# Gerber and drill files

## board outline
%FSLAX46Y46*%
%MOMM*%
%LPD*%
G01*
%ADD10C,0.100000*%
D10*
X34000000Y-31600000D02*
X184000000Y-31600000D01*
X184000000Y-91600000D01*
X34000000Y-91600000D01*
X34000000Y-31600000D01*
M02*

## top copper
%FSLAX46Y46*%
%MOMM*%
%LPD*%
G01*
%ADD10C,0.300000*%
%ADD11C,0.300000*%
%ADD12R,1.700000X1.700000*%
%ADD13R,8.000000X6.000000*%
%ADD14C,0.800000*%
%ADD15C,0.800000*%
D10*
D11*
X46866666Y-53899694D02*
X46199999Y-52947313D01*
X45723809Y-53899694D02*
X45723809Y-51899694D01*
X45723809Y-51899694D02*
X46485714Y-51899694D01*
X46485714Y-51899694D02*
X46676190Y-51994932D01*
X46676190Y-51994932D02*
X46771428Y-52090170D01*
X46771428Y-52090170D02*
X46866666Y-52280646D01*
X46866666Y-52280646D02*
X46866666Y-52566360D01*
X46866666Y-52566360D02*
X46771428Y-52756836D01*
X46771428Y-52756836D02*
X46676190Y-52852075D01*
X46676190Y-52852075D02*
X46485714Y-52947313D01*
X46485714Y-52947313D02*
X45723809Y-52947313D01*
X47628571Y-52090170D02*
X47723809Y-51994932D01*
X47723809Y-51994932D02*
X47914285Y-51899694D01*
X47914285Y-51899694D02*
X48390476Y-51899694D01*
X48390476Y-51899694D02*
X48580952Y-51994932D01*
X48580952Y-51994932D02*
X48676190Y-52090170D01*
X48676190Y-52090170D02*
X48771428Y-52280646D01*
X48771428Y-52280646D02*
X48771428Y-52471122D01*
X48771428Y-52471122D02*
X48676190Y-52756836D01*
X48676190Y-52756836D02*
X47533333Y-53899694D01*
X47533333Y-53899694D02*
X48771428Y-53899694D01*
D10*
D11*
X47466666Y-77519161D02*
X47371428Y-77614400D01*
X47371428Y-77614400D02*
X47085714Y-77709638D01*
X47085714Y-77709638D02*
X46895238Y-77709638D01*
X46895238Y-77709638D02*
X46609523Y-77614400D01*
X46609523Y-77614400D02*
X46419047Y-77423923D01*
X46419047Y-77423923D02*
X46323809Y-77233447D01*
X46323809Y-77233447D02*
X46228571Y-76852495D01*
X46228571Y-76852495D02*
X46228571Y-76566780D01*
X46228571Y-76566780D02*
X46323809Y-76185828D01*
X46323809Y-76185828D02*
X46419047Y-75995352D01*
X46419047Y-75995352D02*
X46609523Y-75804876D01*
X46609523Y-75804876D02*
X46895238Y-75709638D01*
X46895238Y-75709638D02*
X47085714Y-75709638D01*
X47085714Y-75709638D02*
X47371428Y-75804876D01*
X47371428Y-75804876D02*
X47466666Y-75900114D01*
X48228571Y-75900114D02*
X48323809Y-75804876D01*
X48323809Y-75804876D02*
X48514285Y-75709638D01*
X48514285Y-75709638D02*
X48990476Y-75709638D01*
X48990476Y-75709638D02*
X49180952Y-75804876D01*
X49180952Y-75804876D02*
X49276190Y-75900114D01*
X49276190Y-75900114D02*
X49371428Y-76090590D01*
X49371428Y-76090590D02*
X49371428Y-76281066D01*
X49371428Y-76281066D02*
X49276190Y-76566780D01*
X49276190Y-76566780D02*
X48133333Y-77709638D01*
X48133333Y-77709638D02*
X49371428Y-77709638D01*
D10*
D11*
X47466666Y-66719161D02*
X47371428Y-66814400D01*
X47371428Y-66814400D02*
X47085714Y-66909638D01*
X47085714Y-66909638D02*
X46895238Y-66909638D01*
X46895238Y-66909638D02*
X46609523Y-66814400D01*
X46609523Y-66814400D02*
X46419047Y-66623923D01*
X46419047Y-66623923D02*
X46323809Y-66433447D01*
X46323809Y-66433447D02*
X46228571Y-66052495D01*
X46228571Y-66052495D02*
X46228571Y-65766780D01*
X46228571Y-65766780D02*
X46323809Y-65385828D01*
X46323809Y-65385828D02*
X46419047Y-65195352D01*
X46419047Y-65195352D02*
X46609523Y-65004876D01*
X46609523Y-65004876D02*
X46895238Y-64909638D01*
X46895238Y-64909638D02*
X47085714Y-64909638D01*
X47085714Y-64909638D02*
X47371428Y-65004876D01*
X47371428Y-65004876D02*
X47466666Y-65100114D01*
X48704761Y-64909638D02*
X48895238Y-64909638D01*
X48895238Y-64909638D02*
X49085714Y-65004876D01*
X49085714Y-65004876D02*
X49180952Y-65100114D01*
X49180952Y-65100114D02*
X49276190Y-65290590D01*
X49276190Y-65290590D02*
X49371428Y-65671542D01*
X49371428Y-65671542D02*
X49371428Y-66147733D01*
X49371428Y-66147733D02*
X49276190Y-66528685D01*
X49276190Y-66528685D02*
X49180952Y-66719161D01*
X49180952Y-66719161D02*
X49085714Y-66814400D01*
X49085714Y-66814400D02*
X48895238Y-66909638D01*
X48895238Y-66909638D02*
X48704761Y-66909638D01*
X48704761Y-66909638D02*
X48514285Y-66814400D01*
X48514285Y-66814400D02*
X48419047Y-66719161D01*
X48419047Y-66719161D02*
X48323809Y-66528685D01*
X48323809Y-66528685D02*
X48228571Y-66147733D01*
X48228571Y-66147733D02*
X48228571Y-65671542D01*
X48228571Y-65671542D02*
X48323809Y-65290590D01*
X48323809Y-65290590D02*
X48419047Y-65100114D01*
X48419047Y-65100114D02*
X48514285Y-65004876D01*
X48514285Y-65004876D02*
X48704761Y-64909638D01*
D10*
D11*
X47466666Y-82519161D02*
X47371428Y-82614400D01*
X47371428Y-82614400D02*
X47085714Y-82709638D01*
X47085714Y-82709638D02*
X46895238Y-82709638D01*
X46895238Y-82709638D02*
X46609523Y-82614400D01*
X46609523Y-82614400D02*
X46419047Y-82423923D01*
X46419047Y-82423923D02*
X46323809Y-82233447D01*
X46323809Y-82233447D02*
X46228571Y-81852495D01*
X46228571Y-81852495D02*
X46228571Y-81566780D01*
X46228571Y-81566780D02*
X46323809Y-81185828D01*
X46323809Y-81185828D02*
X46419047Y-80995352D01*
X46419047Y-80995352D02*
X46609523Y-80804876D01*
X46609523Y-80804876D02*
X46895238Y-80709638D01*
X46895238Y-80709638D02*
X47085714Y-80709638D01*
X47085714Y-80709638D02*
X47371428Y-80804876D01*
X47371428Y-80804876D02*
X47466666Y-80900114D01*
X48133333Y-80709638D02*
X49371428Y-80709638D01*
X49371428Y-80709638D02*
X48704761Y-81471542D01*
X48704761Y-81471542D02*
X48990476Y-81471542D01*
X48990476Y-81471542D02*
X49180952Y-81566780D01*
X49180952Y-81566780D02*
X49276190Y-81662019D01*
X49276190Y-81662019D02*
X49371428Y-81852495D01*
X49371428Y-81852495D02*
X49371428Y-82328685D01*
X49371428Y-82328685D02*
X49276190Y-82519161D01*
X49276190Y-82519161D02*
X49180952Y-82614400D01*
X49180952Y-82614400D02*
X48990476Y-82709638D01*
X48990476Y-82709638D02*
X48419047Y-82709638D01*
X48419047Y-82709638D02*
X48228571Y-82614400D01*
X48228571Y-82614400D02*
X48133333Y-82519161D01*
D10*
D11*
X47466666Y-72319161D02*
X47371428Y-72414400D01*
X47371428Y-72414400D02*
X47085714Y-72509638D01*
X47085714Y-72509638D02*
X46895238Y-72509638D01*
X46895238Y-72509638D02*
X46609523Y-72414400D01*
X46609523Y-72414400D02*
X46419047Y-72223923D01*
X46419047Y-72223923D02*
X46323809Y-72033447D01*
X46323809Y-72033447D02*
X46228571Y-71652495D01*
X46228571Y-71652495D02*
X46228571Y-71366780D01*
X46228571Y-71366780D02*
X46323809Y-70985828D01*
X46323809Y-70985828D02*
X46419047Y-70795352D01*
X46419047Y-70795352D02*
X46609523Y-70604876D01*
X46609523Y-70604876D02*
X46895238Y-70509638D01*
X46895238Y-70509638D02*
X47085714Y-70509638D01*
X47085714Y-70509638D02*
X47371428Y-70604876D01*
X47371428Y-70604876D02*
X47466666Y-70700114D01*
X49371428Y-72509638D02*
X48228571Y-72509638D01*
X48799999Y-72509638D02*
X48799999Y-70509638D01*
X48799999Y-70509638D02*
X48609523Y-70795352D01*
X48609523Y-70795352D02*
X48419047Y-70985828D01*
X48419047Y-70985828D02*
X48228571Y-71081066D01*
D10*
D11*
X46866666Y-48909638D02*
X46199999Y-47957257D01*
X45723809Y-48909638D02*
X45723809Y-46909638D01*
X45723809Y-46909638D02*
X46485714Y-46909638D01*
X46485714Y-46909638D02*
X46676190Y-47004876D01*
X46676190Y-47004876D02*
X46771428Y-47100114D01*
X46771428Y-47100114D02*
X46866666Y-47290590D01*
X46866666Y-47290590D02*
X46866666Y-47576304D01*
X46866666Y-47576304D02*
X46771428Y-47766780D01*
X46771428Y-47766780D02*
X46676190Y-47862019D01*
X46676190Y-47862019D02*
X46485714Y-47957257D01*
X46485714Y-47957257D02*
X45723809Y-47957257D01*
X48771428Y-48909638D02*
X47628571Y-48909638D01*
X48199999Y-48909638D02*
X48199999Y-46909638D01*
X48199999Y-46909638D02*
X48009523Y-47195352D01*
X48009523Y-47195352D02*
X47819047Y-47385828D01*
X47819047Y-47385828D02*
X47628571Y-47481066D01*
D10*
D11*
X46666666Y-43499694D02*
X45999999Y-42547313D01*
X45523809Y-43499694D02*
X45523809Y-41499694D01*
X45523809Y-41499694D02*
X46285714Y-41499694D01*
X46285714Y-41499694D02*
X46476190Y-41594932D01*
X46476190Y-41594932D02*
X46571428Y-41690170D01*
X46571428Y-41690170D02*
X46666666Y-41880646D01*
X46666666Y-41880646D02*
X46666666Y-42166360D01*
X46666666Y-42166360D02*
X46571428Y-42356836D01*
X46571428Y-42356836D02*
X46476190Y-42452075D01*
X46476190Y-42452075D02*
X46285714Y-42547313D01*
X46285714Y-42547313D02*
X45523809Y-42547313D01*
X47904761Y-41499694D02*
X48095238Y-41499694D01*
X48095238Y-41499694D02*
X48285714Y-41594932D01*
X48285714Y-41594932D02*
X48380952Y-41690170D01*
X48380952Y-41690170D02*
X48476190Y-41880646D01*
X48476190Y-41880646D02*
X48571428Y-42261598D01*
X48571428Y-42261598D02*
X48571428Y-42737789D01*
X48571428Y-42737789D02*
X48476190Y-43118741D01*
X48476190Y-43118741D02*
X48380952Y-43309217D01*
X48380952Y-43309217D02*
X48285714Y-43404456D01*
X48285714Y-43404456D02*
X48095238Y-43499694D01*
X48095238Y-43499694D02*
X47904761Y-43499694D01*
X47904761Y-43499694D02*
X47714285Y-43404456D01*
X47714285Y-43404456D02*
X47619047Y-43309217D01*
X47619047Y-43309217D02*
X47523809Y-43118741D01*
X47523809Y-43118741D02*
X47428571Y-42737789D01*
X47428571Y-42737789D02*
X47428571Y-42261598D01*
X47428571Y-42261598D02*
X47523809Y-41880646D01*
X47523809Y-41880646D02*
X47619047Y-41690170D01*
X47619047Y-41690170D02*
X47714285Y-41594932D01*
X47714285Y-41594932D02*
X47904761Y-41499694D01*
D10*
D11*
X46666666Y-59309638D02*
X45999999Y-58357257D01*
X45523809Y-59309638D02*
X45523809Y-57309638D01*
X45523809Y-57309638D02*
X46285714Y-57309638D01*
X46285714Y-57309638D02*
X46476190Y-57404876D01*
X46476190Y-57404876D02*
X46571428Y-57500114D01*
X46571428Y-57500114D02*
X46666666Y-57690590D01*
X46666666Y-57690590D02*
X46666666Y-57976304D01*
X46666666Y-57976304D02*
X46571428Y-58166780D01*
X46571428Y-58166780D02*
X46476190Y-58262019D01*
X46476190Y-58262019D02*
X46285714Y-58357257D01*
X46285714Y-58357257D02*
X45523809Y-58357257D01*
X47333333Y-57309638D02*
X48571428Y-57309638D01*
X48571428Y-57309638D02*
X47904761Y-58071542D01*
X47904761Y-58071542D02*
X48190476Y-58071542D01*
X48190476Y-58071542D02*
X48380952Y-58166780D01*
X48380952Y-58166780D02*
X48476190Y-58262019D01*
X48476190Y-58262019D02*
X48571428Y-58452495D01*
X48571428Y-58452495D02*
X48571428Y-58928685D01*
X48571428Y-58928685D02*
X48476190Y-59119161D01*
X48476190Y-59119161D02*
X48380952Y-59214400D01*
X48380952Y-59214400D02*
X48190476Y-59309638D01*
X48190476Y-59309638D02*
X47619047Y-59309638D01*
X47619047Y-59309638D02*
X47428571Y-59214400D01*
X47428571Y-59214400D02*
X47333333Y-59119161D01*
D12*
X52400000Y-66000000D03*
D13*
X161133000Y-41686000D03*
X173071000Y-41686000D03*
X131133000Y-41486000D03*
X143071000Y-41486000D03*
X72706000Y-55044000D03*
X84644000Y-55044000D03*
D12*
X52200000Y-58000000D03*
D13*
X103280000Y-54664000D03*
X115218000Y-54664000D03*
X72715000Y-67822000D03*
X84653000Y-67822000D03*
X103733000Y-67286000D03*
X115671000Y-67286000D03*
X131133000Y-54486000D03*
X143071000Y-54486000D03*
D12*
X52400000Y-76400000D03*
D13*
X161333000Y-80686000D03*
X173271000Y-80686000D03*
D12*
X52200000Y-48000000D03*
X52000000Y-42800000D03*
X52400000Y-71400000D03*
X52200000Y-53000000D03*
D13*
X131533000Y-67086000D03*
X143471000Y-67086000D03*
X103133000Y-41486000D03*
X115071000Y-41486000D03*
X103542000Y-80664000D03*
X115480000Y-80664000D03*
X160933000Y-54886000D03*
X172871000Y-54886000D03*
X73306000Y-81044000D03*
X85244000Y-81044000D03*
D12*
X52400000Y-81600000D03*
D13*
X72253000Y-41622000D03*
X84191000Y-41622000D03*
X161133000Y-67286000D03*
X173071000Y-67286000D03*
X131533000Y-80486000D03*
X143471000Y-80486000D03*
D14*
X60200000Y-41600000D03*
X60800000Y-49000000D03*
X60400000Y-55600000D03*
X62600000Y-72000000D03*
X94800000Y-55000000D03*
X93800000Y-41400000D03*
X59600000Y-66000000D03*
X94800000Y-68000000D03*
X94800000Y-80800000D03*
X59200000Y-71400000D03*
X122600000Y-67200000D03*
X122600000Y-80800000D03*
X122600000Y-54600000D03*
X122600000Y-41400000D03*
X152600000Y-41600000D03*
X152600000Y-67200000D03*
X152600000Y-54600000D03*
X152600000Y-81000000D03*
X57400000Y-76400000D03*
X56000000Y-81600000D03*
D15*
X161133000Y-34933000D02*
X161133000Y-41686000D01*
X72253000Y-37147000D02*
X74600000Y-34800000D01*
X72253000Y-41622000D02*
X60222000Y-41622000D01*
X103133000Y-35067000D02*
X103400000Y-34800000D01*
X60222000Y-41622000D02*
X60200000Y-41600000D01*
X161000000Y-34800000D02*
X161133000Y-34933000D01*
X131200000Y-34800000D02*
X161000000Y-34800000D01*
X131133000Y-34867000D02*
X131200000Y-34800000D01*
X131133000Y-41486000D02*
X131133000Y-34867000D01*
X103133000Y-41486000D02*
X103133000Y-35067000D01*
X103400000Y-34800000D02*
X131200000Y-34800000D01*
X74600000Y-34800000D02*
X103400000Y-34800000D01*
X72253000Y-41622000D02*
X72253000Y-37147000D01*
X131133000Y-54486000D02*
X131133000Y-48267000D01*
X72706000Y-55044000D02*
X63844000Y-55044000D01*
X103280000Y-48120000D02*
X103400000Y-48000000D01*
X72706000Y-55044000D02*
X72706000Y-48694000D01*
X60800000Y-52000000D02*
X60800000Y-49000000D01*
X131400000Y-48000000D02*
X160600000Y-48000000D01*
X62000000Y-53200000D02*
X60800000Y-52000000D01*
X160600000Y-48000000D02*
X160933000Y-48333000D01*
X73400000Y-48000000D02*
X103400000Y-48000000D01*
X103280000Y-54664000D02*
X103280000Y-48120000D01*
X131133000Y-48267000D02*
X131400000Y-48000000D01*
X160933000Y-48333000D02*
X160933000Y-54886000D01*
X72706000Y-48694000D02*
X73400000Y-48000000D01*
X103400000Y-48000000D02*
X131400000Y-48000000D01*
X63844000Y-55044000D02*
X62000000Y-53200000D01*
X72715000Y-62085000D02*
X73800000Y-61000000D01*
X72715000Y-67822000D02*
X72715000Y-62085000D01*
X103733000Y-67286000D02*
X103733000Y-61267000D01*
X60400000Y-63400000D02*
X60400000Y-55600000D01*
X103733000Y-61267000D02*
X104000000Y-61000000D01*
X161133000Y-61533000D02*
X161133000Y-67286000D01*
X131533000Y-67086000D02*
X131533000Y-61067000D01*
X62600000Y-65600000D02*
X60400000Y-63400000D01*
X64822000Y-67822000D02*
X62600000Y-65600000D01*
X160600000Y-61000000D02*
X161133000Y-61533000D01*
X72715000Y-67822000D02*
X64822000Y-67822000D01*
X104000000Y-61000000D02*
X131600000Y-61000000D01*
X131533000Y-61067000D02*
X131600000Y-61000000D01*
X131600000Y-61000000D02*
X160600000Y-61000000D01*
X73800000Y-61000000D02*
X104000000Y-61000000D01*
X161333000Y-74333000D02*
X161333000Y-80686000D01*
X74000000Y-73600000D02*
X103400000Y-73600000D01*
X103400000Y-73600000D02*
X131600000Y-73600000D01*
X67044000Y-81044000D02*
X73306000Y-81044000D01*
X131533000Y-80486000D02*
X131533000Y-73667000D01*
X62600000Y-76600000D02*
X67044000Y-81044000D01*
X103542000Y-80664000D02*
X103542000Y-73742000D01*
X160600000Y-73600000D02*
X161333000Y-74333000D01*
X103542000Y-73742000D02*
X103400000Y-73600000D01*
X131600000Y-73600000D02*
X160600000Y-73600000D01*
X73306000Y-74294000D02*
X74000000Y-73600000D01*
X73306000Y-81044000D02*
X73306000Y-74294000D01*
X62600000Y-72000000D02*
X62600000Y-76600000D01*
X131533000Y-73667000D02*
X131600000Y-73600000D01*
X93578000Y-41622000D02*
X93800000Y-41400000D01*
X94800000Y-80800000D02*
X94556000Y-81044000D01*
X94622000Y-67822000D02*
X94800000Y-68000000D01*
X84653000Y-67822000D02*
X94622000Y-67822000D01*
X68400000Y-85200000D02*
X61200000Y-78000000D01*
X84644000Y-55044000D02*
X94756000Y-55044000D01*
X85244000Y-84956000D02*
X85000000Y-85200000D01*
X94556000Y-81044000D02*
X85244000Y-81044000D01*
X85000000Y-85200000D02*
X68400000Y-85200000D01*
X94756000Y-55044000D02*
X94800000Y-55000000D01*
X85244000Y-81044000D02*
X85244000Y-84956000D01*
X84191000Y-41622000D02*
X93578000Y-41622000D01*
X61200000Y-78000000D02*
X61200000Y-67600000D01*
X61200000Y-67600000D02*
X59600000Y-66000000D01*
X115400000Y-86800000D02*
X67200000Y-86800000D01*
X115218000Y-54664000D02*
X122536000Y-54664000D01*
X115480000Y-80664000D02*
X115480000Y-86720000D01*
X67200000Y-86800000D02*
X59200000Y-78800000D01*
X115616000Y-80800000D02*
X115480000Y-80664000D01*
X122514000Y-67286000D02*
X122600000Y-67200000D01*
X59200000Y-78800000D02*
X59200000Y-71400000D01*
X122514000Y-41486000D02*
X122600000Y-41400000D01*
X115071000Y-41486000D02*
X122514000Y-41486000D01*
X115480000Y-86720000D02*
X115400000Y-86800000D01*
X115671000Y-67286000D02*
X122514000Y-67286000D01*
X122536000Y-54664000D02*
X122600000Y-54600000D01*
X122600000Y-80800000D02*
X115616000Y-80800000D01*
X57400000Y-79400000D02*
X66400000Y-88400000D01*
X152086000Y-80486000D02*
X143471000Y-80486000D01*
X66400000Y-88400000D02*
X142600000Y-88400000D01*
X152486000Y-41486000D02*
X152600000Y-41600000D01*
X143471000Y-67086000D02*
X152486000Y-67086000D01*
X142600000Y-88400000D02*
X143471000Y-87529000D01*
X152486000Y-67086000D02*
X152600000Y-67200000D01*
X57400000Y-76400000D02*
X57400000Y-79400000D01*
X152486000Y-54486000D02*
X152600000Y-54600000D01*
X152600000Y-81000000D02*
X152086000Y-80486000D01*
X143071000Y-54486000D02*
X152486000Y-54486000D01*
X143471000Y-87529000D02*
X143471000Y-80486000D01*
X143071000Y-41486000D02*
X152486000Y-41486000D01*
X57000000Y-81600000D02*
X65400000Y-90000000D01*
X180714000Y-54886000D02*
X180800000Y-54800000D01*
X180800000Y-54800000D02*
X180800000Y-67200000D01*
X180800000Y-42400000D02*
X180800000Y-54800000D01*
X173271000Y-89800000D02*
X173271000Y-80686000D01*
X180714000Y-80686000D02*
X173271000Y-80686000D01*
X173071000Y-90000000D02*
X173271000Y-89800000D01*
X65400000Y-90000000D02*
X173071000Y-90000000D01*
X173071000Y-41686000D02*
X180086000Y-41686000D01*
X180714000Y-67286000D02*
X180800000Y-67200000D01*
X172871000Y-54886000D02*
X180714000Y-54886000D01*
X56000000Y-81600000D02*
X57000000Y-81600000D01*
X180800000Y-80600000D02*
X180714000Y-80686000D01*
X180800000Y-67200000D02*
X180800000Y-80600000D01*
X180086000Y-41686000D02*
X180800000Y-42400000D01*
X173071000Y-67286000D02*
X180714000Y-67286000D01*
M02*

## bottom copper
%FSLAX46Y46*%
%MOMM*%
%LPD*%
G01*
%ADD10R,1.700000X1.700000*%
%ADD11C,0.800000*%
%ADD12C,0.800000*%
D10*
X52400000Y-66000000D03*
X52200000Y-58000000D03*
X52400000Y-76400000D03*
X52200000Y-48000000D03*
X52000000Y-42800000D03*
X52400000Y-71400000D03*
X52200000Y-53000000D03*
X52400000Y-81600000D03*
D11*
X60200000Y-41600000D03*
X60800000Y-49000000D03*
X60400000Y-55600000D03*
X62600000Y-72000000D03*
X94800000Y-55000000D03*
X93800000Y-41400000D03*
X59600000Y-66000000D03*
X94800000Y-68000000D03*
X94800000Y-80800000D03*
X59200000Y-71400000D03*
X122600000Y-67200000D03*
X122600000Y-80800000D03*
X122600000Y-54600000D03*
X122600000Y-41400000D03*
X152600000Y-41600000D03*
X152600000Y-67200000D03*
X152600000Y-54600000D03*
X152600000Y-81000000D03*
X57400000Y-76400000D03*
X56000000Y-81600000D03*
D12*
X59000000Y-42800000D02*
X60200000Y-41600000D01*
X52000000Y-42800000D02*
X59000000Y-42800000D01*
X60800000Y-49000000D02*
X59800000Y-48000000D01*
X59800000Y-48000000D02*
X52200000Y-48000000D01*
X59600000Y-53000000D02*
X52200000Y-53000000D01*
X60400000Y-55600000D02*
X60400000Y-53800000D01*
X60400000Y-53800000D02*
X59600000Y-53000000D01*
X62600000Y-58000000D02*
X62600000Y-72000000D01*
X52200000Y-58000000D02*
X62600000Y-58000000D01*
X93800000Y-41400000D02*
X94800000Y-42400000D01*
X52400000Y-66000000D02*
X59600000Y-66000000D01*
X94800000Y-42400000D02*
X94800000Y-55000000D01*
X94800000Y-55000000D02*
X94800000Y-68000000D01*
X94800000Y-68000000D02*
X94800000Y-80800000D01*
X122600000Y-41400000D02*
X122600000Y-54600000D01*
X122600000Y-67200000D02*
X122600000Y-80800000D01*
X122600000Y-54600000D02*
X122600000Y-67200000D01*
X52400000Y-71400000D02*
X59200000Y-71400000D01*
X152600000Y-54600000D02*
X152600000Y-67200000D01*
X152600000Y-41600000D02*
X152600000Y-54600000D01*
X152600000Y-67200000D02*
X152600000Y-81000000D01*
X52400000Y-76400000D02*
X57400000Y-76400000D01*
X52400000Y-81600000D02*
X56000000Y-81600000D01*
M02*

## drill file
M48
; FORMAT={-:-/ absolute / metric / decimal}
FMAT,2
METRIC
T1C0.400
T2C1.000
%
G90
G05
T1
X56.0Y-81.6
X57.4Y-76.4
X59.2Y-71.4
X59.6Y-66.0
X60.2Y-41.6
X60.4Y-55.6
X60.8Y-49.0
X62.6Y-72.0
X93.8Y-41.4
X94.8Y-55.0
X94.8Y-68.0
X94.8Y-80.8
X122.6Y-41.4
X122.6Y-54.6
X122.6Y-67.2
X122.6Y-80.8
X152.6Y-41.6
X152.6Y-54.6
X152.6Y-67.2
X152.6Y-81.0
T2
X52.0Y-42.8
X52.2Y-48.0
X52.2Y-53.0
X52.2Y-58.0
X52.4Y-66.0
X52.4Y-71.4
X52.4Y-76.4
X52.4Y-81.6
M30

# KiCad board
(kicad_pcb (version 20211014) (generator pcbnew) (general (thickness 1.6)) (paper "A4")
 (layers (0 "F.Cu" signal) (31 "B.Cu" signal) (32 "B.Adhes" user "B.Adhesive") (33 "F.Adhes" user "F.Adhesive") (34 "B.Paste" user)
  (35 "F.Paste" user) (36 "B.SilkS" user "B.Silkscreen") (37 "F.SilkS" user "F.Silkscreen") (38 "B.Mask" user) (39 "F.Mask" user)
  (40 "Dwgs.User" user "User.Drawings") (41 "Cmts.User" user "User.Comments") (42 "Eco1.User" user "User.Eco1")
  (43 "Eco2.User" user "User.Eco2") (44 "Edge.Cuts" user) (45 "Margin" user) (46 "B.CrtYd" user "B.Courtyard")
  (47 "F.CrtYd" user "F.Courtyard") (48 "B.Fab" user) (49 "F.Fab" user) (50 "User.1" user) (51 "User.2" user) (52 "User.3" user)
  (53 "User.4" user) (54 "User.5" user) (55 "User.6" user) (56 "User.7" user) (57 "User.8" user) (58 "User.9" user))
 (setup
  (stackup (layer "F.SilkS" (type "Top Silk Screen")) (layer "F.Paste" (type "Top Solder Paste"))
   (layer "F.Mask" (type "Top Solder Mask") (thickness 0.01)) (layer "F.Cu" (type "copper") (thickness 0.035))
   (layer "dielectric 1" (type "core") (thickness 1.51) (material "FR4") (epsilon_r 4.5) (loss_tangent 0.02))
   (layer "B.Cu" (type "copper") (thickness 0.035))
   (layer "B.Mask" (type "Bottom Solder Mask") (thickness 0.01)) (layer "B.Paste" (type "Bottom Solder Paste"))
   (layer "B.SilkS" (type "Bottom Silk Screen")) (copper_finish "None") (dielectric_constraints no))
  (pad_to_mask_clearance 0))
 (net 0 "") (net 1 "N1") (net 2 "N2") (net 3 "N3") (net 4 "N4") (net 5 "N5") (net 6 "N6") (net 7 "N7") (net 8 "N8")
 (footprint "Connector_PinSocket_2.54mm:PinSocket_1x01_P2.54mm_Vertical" (layer "F.Cu") (at 52.4 66)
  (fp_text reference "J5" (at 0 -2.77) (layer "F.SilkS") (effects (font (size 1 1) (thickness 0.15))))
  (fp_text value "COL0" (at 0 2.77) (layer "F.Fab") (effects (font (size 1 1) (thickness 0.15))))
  (pad "1" thru_hole rect (at 0 0) (size 1.7 1.7) (drill 1) (layers *.Cu *.Mask) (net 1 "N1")))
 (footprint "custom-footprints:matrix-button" (layer "F.Cu") (at 156.053 37.622)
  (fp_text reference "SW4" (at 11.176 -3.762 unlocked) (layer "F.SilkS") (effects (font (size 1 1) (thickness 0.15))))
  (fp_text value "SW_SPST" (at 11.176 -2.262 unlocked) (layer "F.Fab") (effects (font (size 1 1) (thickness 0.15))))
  (pad "1" smd rect (at 5.08 4.064) (size 8 6) (layers "F.Cu" "F.Paste" "F.Mask") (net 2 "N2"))
  (pad "2" smd rect (at 17.018 4.064) (size 8 6) (layers "F.Cu" "F.Paste" "F.Mask") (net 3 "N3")))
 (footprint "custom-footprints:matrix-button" (layer "F.Cu") (at 126.053 37.422)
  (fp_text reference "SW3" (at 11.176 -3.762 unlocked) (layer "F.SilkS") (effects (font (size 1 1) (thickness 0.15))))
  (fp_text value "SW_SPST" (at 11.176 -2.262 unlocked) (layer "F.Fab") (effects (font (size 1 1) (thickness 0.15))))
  (pad "1" smd rect (at 5.08 4.064) (size 8 6) (layers "F.Cu" "F.Paste" "F.Mask") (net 2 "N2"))
  (pad "2" smd rect (at 17.018 4.064) (size 8 6) (layers "F.Cu" "F.Paste" "F.Mask") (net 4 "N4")))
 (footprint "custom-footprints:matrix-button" (layer "F.Cu") (at 67.626 50.98)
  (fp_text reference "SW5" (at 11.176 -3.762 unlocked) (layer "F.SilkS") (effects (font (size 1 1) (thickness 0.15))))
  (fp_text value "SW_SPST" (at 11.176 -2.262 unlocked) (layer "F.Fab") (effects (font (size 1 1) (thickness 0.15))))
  (pad "1" smd rect (at 5.08 4.064) (size 8 6) (layers "F.Cu" "F.Paste" "F.Mask") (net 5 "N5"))
  (pad "2" smd rect (at 17.018 4.064) (size 8 6) (layers "F.Cu" "F.Paste" "F.Mask") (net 1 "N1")))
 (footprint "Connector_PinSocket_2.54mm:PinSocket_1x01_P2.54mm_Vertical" (layer "F.Cu") (at 52.2 58)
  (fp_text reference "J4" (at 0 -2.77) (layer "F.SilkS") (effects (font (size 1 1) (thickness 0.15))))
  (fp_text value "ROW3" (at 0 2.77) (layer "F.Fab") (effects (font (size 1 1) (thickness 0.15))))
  (pad "1" thru_hole rect (at 0 0) (size 1.7 1.7) (drill 1) (layers *.Cu *.Mask) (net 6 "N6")))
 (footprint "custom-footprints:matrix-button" (layer "F.Cu") (at 98.2 50.6)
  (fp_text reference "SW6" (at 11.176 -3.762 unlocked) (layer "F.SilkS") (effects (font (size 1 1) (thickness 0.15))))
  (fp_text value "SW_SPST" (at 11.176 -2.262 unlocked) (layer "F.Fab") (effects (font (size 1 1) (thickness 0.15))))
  (pad "1" smd rect (at 5.08 4.064) (size 8 6) (layers "F.Cu" "F.Paste" "F.Mask") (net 5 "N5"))
  (pad "2" smd rect (at 17.018 4.064) (size 8 6) (layers "F.Cu" "F.Paste" "F.Mask") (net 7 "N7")))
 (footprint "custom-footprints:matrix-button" (layer "F.Cu") (at 67.635 63.758)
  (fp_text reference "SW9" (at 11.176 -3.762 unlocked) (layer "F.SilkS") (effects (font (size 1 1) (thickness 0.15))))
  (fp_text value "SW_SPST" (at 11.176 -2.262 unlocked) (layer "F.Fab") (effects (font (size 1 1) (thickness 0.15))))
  (pad "1" smd rect (at 5.08 4.064) (size 8 6) (layers "F.Cu" "F.Paste" "F.Mask") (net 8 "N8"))
  (pad "2" smd rect (at 17.018 4.064) (size 8 6) (layers "F.Cu" "F.Paste" "F.Mask") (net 1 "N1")))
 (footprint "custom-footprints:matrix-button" (layer "F.Cu") (at 98.653 63.222)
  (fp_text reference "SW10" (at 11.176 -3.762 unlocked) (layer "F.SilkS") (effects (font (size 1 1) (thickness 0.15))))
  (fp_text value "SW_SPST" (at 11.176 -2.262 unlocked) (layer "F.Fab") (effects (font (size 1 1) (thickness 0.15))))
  (pad "1" smd rect (at 5.08 4.064) (size 8 6) (layers "F.Cu" "F.Paste" "F.Mask") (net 8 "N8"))
  (pad "2" smd rect (at 17.018 4.064) (size 8 6) (layers "F.Cu" "F.Paste" "F.Mask") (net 7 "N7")))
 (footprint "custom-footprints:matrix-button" (layer "F.Cu") (at 126.053 50.422)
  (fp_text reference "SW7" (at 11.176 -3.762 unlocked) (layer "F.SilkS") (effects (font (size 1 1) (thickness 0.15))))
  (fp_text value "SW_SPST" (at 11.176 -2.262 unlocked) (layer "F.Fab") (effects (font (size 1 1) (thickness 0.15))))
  (pad "1" smd rect (at 5.08 4.064) (size 8 6) (layers "F.Cu" "F.Paste" "F.Mask") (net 5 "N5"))
  (pad "2" smd rect (at 17.018 4.064) (size 8 6) (layers "F.Cu" "F.Paste" "F.Mask") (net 4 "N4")))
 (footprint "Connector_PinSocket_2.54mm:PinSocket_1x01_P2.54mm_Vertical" (layer "F.Cu") (at 52.4 76.4)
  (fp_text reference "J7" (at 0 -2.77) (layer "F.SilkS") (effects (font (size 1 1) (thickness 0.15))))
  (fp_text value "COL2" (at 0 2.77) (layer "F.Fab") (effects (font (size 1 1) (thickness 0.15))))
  (pad "1" thru_hole rect (at 0 0) (size 1.7 1.7) (drill 1) (layers *.Cu *.Mask) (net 4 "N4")))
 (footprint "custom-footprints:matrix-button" (layer "F.Cu") (at 156.253 76.622)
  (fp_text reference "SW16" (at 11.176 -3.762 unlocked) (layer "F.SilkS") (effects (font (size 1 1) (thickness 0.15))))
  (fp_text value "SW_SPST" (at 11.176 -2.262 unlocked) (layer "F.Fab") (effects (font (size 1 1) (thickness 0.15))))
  (pad "1" smd rect (at 5.08 4.064) (size 8 6) (layers "F.Cu" "F.Paste" "F.Mask") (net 6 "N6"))
  (pad "2" smd rect (at 17.018 4.064) (size 8 6) (layers "F.Cu" "F.Paste" "F.Mask") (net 3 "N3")))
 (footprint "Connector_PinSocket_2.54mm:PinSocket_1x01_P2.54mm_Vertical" (layer "F.Cu") (at 52.2 48)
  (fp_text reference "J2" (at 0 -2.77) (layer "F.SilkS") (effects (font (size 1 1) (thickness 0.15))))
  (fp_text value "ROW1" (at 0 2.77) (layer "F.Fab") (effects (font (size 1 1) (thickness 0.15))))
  (pad "1" thru_hole rect (at 0 0) (size 1.7 1.7) (drill 1) (layers *.Cu *.Mask) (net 5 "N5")))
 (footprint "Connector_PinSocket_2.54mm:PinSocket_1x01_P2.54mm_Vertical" (layer "F.Cu") (at 52 42.8)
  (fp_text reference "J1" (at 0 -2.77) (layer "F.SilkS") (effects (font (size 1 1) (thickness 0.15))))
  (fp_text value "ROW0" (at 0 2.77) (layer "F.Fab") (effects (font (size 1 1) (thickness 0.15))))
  (pad "1" thru_hole rect (at 0 0) (size 1.7 1.7) (drill 1) (layers *.Cu *.Mask) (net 2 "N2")))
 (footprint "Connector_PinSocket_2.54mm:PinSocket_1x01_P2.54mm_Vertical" (layer "F.Cu") (at 52.4 71.4)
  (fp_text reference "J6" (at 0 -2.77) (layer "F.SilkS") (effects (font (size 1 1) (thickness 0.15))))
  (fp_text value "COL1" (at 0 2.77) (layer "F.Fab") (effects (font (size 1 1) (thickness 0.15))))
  (pad "1" thru_hole rect (at 0 0) (size 1.7 1.7) (drill 1) (layers *.Cu *.Mask) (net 7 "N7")))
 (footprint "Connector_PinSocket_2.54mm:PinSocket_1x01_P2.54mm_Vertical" (layer "F.Cu") (at 52.2 53)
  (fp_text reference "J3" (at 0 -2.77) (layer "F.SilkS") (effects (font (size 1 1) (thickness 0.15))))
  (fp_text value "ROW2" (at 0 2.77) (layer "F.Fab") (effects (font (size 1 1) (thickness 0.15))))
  (pad "1" thru_hole rect (at 0 0) (size 1.7 1.7) (drill 1) (layers *.Cu *.Mask) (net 8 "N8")))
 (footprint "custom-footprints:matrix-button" (layer "F.Cu") (at 126.453 63.022)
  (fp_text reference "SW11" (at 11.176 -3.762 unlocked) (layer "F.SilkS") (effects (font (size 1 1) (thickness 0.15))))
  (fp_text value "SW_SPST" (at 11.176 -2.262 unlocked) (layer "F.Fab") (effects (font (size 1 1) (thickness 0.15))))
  (pad "1" smd rect (at 5.08 4.064) (size 8 6) (layers "F.Cu" "F.Paste" "F.Mask") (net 8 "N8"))
  (pad "2" smd rect (at 17.018 4.064) (size 8 6) (layers "F.Cu" "F.Paste" "F.Mask") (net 4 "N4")))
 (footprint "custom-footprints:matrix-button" (layer "F.Cu") (at 98.053 37.422)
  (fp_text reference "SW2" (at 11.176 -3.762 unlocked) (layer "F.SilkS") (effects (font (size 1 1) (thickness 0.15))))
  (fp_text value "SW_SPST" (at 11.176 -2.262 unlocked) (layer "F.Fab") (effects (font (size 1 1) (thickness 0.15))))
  (pad "1" smd rect (at 5.08 4.064) (size 8 6) (layers "F.Cu" "F.Paste" "F.Mask") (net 2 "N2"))
  (pad "2" smd rect (at 17.018 4.064) (size 8 6) (layers "F.Cu" "F.Paste" "F.Mask") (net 7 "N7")))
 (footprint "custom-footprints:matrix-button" (layer "F.Cu") (at 98.462 76.6)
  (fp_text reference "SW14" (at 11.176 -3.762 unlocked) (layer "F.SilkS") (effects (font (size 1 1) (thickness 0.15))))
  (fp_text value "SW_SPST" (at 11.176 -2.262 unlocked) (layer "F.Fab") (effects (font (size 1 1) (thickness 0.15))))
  (pad "1" smd rect (at 5.08 4.064) (size 8 6) (layers "F.Cu" "F.Paste" "F.Mask") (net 6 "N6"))
  (pad "2" smd rect (at 17.018 4.064) (size 8 6) (layers "F.Cu" "F.Paste" "F.Mask") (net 7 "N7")))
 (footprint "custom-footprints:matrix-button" (layer "F.Cu") (at 155.853 50.822)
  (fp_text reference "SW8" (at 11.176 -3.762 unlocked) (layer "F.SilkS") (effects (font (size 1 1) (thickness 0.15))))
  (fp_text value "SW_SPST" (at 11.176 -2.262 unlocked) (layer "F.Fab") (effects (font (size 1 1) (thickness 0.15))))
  (pad "1" smd rect (at 5.08 4.064) (size 8 6) (layers "F.Cu" "F.Paste" "F.Mask") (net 5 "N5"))
  (pad "2" smd rect (at 17.018 4.064) (size 8 6) (layers "F.Cu" "F.Paste" "F.Mask") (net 3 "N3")))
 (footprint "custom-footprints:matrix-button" (layer "F.Cu") (at 68.226 76.98)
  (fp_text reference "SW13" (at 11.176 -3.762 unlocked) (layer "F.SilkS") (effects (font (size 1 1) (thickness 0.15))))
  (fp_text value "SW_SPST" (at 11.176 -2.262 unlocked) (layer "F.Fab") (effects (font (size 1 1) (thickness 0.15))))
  (pad "1" smd rect (at 5.08 4.064) (size 8 6) (layers "F.Cu" "F.Paste" "F.Mask") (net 6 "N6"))
  (pad "2" smd rect (at 17.018 4.064) (size 8 6) (layers "F.Cu" "F.Paste" "F.Mask") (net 1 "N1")))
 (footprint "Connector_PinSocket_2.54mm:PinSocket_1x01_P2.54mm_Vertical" (layer "F.Cu") (at 52.4 81.6)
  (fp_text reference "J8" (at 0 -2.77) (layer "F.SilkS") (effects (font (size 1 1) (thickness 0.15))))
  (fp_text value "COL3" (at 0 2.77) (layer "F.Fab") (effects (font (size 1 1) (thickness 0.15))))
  (pad "1" thru_hole rect (at 0 0) (size 1.7 1.7) (drill 1) (layers *.Cu *.Mask) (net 3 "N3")))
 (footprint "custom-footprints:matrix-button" (layer "F.Cu") (at 67.173 37.558)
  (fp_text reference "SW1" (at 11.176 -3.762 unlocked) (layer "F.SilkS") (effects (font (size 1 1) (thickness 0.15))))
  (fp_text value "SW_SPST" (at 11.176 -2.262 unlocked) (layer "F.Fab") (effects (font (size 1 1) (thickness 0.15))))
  (pad "1" smd rect (at 5.08 4.064) (size 8 6) (layers "F.Cu" "F.Paste" "F.Mask") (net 2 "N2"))
  (pad "2" smd rect (at 17.018 4.064) (size 8 6) (layers "F.Cu" "F.Paste" "F.Mask") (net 1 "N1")))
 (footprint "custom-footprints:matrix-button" (layer "F.Cu") (at 156.053 63.222)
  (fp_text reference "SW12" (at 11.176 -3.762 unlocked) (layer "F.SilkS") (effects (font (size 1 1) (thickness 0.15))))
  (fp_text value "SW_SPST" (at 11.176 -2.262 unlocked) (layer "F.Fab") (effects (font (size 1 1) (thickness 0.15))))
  (pad "1" smd rect (at 5.08 4.064) (size 8 6) (layers "F.Cu" "F.Paste" "F.Mask") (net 8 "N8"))
  (pad "2" smd rect (at 17.018 4.064) (size 8 6) (layers "F.Cu" "F.Paste" "F.Mask") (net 3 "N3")))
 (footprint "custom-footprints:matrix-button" (layer "F.Cu") (at 126.453 76.422)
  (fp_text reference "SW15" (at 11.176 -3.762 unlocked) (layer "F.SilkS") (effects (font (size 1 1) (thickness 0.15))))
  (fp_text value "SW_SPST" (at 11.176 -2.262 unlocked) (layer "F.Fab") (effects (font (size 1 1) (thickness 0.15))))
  (pad "1" smd rect (at 5.08 4.064) (size 8 6) (layers "F.Cu" "F.Paste" "F.Mask") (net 6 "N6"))
  (pad "2" smd rect (at 17.018 4.064) (size 8 6) (layers "F.Cu" "F.Paste" "F.Mask") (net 4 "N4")))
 (gr_rect (start 34 91.6) (end 184 31.6) (layer "Edge.Cuts") (width 0.1) (fill none))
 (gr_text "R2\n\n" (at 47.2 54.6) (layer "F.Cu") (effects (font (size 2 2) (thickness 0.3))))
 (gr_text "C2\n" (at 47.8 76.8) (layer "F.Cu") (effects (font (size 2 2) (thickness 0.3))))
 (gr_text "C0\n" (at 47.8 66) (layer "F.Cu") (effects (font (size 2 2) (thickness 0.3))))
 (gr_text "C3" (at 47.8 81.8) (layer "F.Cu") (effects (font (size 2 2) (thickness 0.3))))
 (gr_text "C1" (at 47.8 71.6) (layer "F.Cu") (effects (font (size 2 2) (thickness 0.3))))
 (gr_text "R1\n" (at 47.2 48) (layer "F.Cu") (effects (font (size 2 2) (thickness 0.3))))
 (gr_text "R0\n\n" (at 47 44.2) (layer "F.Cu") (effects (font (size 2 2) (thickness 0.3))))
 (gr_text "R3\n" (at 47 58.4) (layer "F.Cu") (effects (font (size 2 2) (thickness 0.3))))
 (segment (start 161.133 34.933) (end 161.133 41.686) (width 0.8) (layer "F.Cu") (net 2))
 (segment (start 72.253 37.147) (end 74.6 34.8) (width 0.8) (layer "F.Cu") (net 2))
 (segment (start 72.253 41.622) (end 60.222 41.622) (width 0.8) (layer "F.Cu") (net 2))
 (segment (start 103.133 35.067) (end 103.4 34.8) (width 0.8) (layer "F.Cu") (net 2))
 (segment (start 60.222 41.622) (end 60.2 41.6) (width 0.8) (layer "F.Cu") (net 2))
 (segment (start 161 34.8) (end 161.133 34.933) (width 0.8) (layer "F.Cu") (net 2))
 (segment (start 131.2 34.8) (end 161 34.8) (width 0.8) (layer "F.Cu") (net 2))
 (segment (start 131.133 34.867) (end 131.2 34.8) (width 0.8) (layer "F.Cu") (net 2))
 (segment (start 131.133 41.486) (end 131.133 34.867) (width 0.8) (layer "F.Cu") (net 2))
 (segment (start 103.133 41.486) (end 103.133 35.067) (width 0.8) (layer "F.Cu") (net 2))
 (segment (start 103.4 34.8) (end 131.2 34.8) (width 0.8) (layer "F.Cu") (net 2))
 (segment (start 74.6 34.8) (end 103.4 34.8) (width 0.8) (layer "F.Cu") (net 2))
 (segment (start 72.253 41.622) (end 72.253 37.147) (width 0.8) (layer "F.Cu") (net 2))
 (via (at 60.2 41.6) (size 0.8) (drill 0.4) (layers "F.Cu" "B.Cu") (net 2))
 (segment (start 59 42.8) (end 60.2 41.6) (width 0.8) (layer "B.Cu") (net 2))
 (segment (start 52 42.8) (end 59 42.8) (width 0.8) (layer "B.Cu") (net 2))
 (segment (start 131.133 54.486) (end 131.133 48.267) (width 0.8) (layer "F.Cu") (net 5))
 (segment (start 72.706 55.044) (end 63.844 55.044) (width 0.8) (layer "F.Cu") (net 5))
 (segment (start 103.28 48.12) (end 103.4 48) (width 0.8) (layer "F.Cu") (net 5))
 (segment (start 72.706 55.044) (end 72.706 48.694) (width 0.8) (layer "F.Cu") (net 5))
 (segment (start 60.8 52) (end 60.8 49) (width 0.8) (layer "F.Cu") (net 5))
 (segment (start 131.4 48) (end 160.6 48) (width 0.8) (layer "F.Cu") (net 5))
 (segment (start 62 53.2) (end 60.8 52) (width 0.8) (layer "F.Cu") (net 5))
 (segment (start 160.6 48) (end 160.933 48.333) (width 0.8) (layer "F.Cu") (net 5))
 (segment (start 73.4 48) (end 103.4 48) (width 0.8) (layer "F.Cu") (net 5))
 (segment (start 103.28 54.664) (end 103.28 48.12) (width 0.8) (layer "F.Cu") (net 5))
 (segment (start 131.133 48.267) (end 131.4 48) (width 0.8) (layer "F.Cu") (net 5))
 (segment (start 160.933 48.333) (end 160.933 54.886) (width 0.8) (layer "F.Cu") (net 5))
 (segment (start 72.706 48.694) (end 73.4 48) (width 0.8) (layer "F.Cu") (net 5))
 (segment (start 103.4 48) (end 131.4 48) (width 0.8) (layer "F.Cu") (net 5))
 (segment (start 63.844 55.044) (end 62 53.2) (width 0.8) (layer "F.Cu") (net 5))
 (via (at 60.8 49) (size 0.8) (drill 0.4) (layers "F.Cu" "B.Cu") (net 5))
 (segment (start 60.8 49) (end 59.8 48) (width 0.8) (layer "B.Cu") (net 5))
 (segment (start 59.8 48) (end 52.2 48) (width 0.8) (layer "B.Cu") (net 5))
 (segment (start 72.715 62.085) (end 73.8 61) (width 0.8) (layer "F.Cu") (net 8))
 (segment (start 72.715 67.822) (end 72.715 62.085) (width 0.8) (layer "F.Cu") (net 8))
 (segment (start 103.733 67.286) (end 103.733 61.267) (width 0.8) (layer "F.Cu") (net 8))
 (segment (start 60.4 63.4) (end 60.4 55.6) (width 0.8) (layer "F.Cu") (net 8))
 (segment (start 103.733 61.267) (end 104 61) (width 0.8) (layer "F.Cu") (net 8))
 (segment (start 161.133 61.533) (end 161.133 67.286) (width 0.8) (layer "F.Cu") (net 8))
 (segment (start 131.533 67.086) (end 131.533 61.067) (width 0.8) (layer "F.Cu") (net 8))
 (segment (start 62.6 65.6) (end 60.4 63.4) (width 0.8) (layer "F.Cu") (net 8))
 (segment (start 64.822 67.822) (end 62.6 65.6) (width 0.8) (layer "F.Cu") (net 8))
 (segment (start 160.6 61) (end 161.133 61.533) (width 0.8) (layer "F.Cu") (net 8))
 (segment (start 72.715 67.822) (end 64.822 67.822) (width 0.8) (layer "F.Cu") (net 8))
 (segment (start 104 61) (end 131.6 61) (width 0.8) (layer "F.Cu") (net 8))
 (segment (start 131.533 61.067) (end 131.6 61) (width 0.8) (layer "F.Cu") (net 8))
 (segment (start 131.6 61) (end 160.6 61) (width 0.8) (layer "F.Cu") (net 8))
 (segment (start 73.8 61) (end 104 61) (width 0.8) (layer "F.Cu") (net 8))
 (via (at 60.4 55.6) (size 0.8) (drill 0.4) (layers "F.Cu" "B.Cu") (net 8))
 (segment (start 59.6 53) (end 52.2 53) (width 0.8) (layer "B.Cu") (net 8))
 (segment (start 60.4 55.6) (end 60.4 53.8) (width 0.8) (layer "B.Cu") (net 8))
 (segment (start 60.4 53.8) (end 59.6 53) (width 0.8) (layer "B.Cu") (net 8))
 (segment (start 161.333 74.333) (end 161.333 80.686) (width 0.8) (layer "F.Cu") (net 6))
 (segment (start 74 73.6) (end 103.4 73.6) (width 0.8) (layer "F.Cu") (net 6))
 (segment (start 103.4 73.6) (end 131.6 73.6) (width 0.8) (layer "F.Cu") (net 6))
 (segment (start 67.044 81.044) (end 73.306 81.044) (width 0.8) (layer "F.Cu") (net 6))
 (segment (start 131.533 80.486) (end 131.533 73.667) (width 0.8) (layer "F.Cu") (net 6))
 (segment (start 62.6 76.6) (end 67.044 81.044) (width 0.8) (layer "F.Cu") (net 6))
 (segment (start 103.542 80.664) (end 103.542 73.742) (width 0.8) (layer "F.Cu") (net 6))
 (segment (start 160.6 73.6) (end 161.333 74.333) (width 0.8) (layer "F.Cu") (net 6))
 (segment (start 103.542 73.742) (end 103.4 73.6) (width 0.8) (layer "F.Cu") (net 6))
 (segment (start 131.6 73.6) (end 160.6 73.6) (width 0.8) (layer "F.Cu") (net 6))
 (segment (start 73.306 74.294) (end 74 73.6) (width 0.8) (layer "F.Cu") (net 6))
 (segment (start 73.306 81.044) (end 73.306 74.294) (width 0.8) (layer "F.Cu") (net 6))
 (segment (start 62.6 72) (end 62.6 76.6) (width 0.8) (layer "F.Cu") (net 6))
 (segment (start 131.533 73.667) (end 131.6 73.6) (width 0.8) (layer "F.Cu") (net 6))
 (via (at 62.6 72) (size 0.8) (drill 0.4) (layers "F.Cu" "B.Cu") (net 6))
 (segment (start 62.6 58) (end 62.6 72) (width 0.8) (layer "B.Cu") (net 6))
 (segment (start 52.2 58) (end 62.6 58) (width 0.8) (layer "B.Cu") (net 6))
 (segment (start 93.578 41.622) (end 93.8 41.4) (width 0.8) (layer "F.Cu") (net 1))
 (segment (start 94.8 80.8) (end 94.556 81.044) (width 0.8) (layer "F.Cu") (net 1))
 (segment (start 94.622 67.822) (end 94.8 68) (width 0.8) (layer "F.Cu") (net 1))
 (segment (start 84.653 67.822) (end 94.622 67.822) (width 0.8) (layer "F.Cu") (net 1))
 (segment (start 68.4 85.2) (end 61.2 78) (width 0.8) (layer "F.Cu") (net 1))
 (segment (start 84.644 55.044) (end 94.756 55.044) (width 0.8) (layer "F.Cu") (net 1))
 (segment (start 85.244 84.956) (end 85 85.2) (width 0.8) (layer "F.Cu") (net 1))
 (segment (start 94.556 81.044) (end 85.244 81.044) (width 0.8) (layer "F.Cu") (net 1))
 (segment (start 85 85.2) (end 68.4 85.2) (width 0.8) (layer "F.Cu") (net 1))
 (segment (start 94.756 55.044) (end 94.8 55) (width 0.8) (layer "F.Cu") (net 1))
 (segment (start 85.244 81.044) (end 85.244 84.956) (width 0.8) (layer "F.Cu") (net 1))
 (segment (start 84.191 41.622) (end 93.578 41.622) (width 0.8) (layer "F.Cu") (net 1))
 (segment (start 61.2 78) (end 61.2 67.6) (width 0.8) (layer "F.Cu") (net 1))
 (segment (start 61.2 67.6) (end 59.6 66) (width 0.8) (layer "F.Cu") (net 1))
 (via (at 94.8 55) (size 0.8) (drill 0.4) (layers "F.Cu" "B.Cu") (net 1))
 (via (at 93.8 41.4) (size 0.8) (drill 0.4) (layers "F.Cu" "B.Cu") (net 1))
 (via (at 59.6 66) (size 0.8) (drill 0.4) (layers "F.Cu" "B.Cu") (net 1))
 (via (at 94.8 68) (size 0.8) (drill 0.4) (layers "F.Cu" "B.Cu") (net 1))
 (via (at 94.8 80.8) (size 0.8) (drill 0.4) (layers "F.Cu" "B.Cu") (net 1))
 (segment (start 93.8 41.4) (end 94.8 42.4) (width 0.8) (layer "B.Cu") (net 1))
 (segment (start 52.4 66) (end 59.6 66) (width 0.8) (layer "B.Cu") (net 1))
 (segment (start 94.8 42.4) (end 94.8 55) (width 0.8) (layer "B.Cu") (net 1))
 (segment (start 94.8 55) (end 94.8 68) (width 0.8) (layer "B.Cu") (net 1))
 (segment (start 94.8 68) (end 94.8 80.8) (width 0.8) (layer "B.Cu") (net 1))
 (segment (start 115.4 86.8) (end 67.2 86.8) (width 0.8) (layer "F.Cu") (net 7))
 (segment (start 115.218 54.664) (end 122.536 54.664) (width 0.8) (layer "F.Cu") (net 7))
 (segment (start 115.48 80.664) (end 115.48 86.72) (width 0.8) (layer "F.Cu") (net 7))
 (segment (start 67.2 86.8) (end 59.2 78.8) (width 0.8) (layer "F.Cu") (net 7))
 (segment (start 115.616 80.8) (end 115.48 80.664) (width 0.8) (layer "F.Cu") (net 7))
 (segment (start 122.514 67.286) (end 122.6 67.2) (width 0.8) (layer "F.Cu") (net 7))
 (segment (start 59.2 78.8) (end 59.2 71.4) (width 0.8) (layer "F.Cu") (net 7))
 (segment (start 122.514 41.486) (end 122.6 41.4) (width 0.8) (layer "F.Cu") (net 7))
 (segment (start 115.071 41.486) (end 122.514 41.486) (width 0.8) (layer "F.Cu") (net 7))
 (segment (start 115.48 86.72) (end 115.4 86.8) (width 0.8) (layer "F.Cu") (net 7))
 (segment (start 115.671 67.286) (end 122.514 67.286) (width 0.8) (layer "F.Cu") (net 7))
 (segment (start 122.536 54.664) (end 122.6 54.6) (width 0.8) (layer "F.Cu") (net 7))
 (segment (start 122.6 80.8) (end 115.616 80.8) (width 0.8) (layer "F.Cu") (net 7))
 (via (at 59.2 71.4) (size 0.8) (drill 0.4) (layers "F.Cu" "B.Cu") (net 7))
 (via (at 122.6 67.2) (size 0.8) (drill 0.4) (layers "F.Cu" "B.Cu") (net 7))
 (via (at 122.6 80.8) (size 0.8) (drill 0.4) (layers "F.Cu" "B.Cu") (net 7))
 (via (at 122.6 54.6) (size 0.8) (drill 0.4) (layers "F.Cu" "B.Cu") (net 7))
 (via (at 122.6 41.4) (size 0.8) (drill 0.4) (layers "F.Cu" "B.Cu") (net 7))
 (segment (start 122.6 41.4) (end 122.6 54.6) (width 0.8) (layer "B.Cu") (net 7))
 (segment (start 122.6 67.2) (end 122.6 80.8) (width 0.8) (layer "B.Cu") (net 7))
 (segment (start 122.6 54.6) (end 122.6 67.2) (width 0.8) (layer "B.Cu") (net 7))
 (segment (start 52.4 71.4) (end 59.2 71.4) (width 0.8) (layer "B.Cu") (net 7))
 (segment (start 57.4 79.4) (end 66.4 88.4) (width 0.8) (layer "F.Cu") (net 4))
 (segment (start 152.086 80.486) (end 143.471 80.486) (width 0.8) (layer "F.Cu") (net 4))
 (segment (start 66.4 88.4) (end 142.6 88.4) (width 0.8) (layer "F.Cu") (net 4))
 (segment (start 152.486 41.486) (end 152.6 41.6) (width 0.8) (layer "F.Cu") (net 4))
 (segment (start 143.471 67.086) (end 152.486 67.086) (width 0.8) (layer "F.Cu") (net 4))
 (segment (start 142.6 88.4) (end 143.471 87.529) (width 0.8) (layer "F.Cu") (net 4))
 (segment (start 152.486 67.086) (end 152.6 67.2) (width 0.8) (layer "F.Cu") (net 4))
 (segment (start 57.4 76.4) (end 57.4 79.4) (width 0.8) (layer "F.Cu") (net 4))
 (segment (start 152.486 54.486) (end 152.6 54.6) (width 0.8) (layer "F.Cu") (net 4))
 (segment (start 152.6 81) (end 152.086 80.486) (width 0.8) (layer "F.Cu") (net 4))
 (segment (start 143.071 54.486) (end 152.486 54.486) (width 0.8) (layer "F.Cu") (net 4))
 (segment (start 143.471 87.529) (end 143.471 80.486) (width 0.8) (layer "F.Cu") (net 4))
 (segment (start 143.071 41.486) (end 152.486 41.486) (width 0.8) (layer "F.Cu") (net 4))
 (via (at 152.6 41.6) (size 0.8) (drill 0.4) (layers "F.Cu" "B.Cu") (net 4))
 (via (at 152.6 67.2) (size 0.8) (drill 0.4) (layers "F.Cu" "B.Cu") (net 4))
 (via (at 152.6 54.6) (size 0.8) (drill 0.4) (layers "F.Cu" "B.Cu") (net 4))
 (via (at 152.6 81) (size 0.8) (drill 0.4) (layers "F.Cu" "B.Cu") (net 4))
 (via (at 57.4 76.4) (size 0.8) (drill 0.4) (layers "F.Cu" "B.Cu") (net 4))
 (segment (start 152.6 54.6) (end 152.6 67.2) (width 0.8) (layer "B.Cu") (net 4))
 (segment (start 152.6 41.6) (end 152.6 54.6) (width 0.8) (layer "B.Cu") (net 4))
 (segment (start 152.6 67.2) (end 152.6 81) (width 0.8) (layer "B.Cu") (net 4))
 (segment (start 52.4 76.4) (end 57.4 76.4) (width 0.8) (layer "B.Cu") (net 4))
 (segment (start 57 81.6) (end 65.4 90) (width 0.8) (layer "F.Cu") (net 3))
 (segment (start 180.714 54.886) (end 180.8 54.8) (width 0.8) (layer "F.Cu") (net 3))
 (segment (start 180.8 54.8) (end 180.8 67.2) (width 0.8) (layer "F.Cu") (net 3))
 (segment (start 180.8 42.4) (end 180.8 54.8) (width 0.8) (layer "F.Cu") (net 3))
 (segment (start 173.271 89.8) (end 173.271 80.686) (width 0.8) (layer "F.Cu") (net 3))
 (segment (start 180.714 80.686) (end 173.271 80.686) (width 0.8) (layer "F.Cu") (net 3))
 (segment (start 173.071 90) (end 173.271 89.8) (width 0.8) (layer "F.Cu") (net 3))
 (segment (start 65.4 90) (end 173.071 90) (width 0.8) (layer "F.Cu") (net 3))
 (segment (start 173.071 41.686) (end 180.086 41.686) (width 0.8) (layer "F.Cu") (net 3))
 (segment (start 180.714 67.286) (end 180.8 67.2) (width 0.8) (layer "F.Cu") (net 3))
 (segment (start 172.871 54.886) (end 180.714 54.886) (width 0.8) (layer "F.Cu") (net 3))
 (segment (start 56 81.6) (end 57 81.6) (width 0.8) (layer "F.Cu") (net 3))
 (segment (start 180.8 80.6) (end 180.714 80.686) (width 0.8) (layer "F.Cu") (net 3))
 (segment (start 180.8 67.2) (end 180.8 80.6) (width 0.8) (layer "F.Cu") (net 3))
 (segment (start 180.086 41.686) (end 180.8 42.4) (width 0.8) (layer "F.Cu") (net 3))
 (segment (start 173.071 67.286) (end 180.714 67.286) (width 0.8) (layer "F.Cu") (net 3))
 (via (at 56 81.6) (size 0.8) (drill 0.4) (layers "F.Cu" "B.Cu") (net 3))
 (segment (start 52.4 81.6) (end 56 81.6) (width 0.8) (layer "B.Cu") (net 3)))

